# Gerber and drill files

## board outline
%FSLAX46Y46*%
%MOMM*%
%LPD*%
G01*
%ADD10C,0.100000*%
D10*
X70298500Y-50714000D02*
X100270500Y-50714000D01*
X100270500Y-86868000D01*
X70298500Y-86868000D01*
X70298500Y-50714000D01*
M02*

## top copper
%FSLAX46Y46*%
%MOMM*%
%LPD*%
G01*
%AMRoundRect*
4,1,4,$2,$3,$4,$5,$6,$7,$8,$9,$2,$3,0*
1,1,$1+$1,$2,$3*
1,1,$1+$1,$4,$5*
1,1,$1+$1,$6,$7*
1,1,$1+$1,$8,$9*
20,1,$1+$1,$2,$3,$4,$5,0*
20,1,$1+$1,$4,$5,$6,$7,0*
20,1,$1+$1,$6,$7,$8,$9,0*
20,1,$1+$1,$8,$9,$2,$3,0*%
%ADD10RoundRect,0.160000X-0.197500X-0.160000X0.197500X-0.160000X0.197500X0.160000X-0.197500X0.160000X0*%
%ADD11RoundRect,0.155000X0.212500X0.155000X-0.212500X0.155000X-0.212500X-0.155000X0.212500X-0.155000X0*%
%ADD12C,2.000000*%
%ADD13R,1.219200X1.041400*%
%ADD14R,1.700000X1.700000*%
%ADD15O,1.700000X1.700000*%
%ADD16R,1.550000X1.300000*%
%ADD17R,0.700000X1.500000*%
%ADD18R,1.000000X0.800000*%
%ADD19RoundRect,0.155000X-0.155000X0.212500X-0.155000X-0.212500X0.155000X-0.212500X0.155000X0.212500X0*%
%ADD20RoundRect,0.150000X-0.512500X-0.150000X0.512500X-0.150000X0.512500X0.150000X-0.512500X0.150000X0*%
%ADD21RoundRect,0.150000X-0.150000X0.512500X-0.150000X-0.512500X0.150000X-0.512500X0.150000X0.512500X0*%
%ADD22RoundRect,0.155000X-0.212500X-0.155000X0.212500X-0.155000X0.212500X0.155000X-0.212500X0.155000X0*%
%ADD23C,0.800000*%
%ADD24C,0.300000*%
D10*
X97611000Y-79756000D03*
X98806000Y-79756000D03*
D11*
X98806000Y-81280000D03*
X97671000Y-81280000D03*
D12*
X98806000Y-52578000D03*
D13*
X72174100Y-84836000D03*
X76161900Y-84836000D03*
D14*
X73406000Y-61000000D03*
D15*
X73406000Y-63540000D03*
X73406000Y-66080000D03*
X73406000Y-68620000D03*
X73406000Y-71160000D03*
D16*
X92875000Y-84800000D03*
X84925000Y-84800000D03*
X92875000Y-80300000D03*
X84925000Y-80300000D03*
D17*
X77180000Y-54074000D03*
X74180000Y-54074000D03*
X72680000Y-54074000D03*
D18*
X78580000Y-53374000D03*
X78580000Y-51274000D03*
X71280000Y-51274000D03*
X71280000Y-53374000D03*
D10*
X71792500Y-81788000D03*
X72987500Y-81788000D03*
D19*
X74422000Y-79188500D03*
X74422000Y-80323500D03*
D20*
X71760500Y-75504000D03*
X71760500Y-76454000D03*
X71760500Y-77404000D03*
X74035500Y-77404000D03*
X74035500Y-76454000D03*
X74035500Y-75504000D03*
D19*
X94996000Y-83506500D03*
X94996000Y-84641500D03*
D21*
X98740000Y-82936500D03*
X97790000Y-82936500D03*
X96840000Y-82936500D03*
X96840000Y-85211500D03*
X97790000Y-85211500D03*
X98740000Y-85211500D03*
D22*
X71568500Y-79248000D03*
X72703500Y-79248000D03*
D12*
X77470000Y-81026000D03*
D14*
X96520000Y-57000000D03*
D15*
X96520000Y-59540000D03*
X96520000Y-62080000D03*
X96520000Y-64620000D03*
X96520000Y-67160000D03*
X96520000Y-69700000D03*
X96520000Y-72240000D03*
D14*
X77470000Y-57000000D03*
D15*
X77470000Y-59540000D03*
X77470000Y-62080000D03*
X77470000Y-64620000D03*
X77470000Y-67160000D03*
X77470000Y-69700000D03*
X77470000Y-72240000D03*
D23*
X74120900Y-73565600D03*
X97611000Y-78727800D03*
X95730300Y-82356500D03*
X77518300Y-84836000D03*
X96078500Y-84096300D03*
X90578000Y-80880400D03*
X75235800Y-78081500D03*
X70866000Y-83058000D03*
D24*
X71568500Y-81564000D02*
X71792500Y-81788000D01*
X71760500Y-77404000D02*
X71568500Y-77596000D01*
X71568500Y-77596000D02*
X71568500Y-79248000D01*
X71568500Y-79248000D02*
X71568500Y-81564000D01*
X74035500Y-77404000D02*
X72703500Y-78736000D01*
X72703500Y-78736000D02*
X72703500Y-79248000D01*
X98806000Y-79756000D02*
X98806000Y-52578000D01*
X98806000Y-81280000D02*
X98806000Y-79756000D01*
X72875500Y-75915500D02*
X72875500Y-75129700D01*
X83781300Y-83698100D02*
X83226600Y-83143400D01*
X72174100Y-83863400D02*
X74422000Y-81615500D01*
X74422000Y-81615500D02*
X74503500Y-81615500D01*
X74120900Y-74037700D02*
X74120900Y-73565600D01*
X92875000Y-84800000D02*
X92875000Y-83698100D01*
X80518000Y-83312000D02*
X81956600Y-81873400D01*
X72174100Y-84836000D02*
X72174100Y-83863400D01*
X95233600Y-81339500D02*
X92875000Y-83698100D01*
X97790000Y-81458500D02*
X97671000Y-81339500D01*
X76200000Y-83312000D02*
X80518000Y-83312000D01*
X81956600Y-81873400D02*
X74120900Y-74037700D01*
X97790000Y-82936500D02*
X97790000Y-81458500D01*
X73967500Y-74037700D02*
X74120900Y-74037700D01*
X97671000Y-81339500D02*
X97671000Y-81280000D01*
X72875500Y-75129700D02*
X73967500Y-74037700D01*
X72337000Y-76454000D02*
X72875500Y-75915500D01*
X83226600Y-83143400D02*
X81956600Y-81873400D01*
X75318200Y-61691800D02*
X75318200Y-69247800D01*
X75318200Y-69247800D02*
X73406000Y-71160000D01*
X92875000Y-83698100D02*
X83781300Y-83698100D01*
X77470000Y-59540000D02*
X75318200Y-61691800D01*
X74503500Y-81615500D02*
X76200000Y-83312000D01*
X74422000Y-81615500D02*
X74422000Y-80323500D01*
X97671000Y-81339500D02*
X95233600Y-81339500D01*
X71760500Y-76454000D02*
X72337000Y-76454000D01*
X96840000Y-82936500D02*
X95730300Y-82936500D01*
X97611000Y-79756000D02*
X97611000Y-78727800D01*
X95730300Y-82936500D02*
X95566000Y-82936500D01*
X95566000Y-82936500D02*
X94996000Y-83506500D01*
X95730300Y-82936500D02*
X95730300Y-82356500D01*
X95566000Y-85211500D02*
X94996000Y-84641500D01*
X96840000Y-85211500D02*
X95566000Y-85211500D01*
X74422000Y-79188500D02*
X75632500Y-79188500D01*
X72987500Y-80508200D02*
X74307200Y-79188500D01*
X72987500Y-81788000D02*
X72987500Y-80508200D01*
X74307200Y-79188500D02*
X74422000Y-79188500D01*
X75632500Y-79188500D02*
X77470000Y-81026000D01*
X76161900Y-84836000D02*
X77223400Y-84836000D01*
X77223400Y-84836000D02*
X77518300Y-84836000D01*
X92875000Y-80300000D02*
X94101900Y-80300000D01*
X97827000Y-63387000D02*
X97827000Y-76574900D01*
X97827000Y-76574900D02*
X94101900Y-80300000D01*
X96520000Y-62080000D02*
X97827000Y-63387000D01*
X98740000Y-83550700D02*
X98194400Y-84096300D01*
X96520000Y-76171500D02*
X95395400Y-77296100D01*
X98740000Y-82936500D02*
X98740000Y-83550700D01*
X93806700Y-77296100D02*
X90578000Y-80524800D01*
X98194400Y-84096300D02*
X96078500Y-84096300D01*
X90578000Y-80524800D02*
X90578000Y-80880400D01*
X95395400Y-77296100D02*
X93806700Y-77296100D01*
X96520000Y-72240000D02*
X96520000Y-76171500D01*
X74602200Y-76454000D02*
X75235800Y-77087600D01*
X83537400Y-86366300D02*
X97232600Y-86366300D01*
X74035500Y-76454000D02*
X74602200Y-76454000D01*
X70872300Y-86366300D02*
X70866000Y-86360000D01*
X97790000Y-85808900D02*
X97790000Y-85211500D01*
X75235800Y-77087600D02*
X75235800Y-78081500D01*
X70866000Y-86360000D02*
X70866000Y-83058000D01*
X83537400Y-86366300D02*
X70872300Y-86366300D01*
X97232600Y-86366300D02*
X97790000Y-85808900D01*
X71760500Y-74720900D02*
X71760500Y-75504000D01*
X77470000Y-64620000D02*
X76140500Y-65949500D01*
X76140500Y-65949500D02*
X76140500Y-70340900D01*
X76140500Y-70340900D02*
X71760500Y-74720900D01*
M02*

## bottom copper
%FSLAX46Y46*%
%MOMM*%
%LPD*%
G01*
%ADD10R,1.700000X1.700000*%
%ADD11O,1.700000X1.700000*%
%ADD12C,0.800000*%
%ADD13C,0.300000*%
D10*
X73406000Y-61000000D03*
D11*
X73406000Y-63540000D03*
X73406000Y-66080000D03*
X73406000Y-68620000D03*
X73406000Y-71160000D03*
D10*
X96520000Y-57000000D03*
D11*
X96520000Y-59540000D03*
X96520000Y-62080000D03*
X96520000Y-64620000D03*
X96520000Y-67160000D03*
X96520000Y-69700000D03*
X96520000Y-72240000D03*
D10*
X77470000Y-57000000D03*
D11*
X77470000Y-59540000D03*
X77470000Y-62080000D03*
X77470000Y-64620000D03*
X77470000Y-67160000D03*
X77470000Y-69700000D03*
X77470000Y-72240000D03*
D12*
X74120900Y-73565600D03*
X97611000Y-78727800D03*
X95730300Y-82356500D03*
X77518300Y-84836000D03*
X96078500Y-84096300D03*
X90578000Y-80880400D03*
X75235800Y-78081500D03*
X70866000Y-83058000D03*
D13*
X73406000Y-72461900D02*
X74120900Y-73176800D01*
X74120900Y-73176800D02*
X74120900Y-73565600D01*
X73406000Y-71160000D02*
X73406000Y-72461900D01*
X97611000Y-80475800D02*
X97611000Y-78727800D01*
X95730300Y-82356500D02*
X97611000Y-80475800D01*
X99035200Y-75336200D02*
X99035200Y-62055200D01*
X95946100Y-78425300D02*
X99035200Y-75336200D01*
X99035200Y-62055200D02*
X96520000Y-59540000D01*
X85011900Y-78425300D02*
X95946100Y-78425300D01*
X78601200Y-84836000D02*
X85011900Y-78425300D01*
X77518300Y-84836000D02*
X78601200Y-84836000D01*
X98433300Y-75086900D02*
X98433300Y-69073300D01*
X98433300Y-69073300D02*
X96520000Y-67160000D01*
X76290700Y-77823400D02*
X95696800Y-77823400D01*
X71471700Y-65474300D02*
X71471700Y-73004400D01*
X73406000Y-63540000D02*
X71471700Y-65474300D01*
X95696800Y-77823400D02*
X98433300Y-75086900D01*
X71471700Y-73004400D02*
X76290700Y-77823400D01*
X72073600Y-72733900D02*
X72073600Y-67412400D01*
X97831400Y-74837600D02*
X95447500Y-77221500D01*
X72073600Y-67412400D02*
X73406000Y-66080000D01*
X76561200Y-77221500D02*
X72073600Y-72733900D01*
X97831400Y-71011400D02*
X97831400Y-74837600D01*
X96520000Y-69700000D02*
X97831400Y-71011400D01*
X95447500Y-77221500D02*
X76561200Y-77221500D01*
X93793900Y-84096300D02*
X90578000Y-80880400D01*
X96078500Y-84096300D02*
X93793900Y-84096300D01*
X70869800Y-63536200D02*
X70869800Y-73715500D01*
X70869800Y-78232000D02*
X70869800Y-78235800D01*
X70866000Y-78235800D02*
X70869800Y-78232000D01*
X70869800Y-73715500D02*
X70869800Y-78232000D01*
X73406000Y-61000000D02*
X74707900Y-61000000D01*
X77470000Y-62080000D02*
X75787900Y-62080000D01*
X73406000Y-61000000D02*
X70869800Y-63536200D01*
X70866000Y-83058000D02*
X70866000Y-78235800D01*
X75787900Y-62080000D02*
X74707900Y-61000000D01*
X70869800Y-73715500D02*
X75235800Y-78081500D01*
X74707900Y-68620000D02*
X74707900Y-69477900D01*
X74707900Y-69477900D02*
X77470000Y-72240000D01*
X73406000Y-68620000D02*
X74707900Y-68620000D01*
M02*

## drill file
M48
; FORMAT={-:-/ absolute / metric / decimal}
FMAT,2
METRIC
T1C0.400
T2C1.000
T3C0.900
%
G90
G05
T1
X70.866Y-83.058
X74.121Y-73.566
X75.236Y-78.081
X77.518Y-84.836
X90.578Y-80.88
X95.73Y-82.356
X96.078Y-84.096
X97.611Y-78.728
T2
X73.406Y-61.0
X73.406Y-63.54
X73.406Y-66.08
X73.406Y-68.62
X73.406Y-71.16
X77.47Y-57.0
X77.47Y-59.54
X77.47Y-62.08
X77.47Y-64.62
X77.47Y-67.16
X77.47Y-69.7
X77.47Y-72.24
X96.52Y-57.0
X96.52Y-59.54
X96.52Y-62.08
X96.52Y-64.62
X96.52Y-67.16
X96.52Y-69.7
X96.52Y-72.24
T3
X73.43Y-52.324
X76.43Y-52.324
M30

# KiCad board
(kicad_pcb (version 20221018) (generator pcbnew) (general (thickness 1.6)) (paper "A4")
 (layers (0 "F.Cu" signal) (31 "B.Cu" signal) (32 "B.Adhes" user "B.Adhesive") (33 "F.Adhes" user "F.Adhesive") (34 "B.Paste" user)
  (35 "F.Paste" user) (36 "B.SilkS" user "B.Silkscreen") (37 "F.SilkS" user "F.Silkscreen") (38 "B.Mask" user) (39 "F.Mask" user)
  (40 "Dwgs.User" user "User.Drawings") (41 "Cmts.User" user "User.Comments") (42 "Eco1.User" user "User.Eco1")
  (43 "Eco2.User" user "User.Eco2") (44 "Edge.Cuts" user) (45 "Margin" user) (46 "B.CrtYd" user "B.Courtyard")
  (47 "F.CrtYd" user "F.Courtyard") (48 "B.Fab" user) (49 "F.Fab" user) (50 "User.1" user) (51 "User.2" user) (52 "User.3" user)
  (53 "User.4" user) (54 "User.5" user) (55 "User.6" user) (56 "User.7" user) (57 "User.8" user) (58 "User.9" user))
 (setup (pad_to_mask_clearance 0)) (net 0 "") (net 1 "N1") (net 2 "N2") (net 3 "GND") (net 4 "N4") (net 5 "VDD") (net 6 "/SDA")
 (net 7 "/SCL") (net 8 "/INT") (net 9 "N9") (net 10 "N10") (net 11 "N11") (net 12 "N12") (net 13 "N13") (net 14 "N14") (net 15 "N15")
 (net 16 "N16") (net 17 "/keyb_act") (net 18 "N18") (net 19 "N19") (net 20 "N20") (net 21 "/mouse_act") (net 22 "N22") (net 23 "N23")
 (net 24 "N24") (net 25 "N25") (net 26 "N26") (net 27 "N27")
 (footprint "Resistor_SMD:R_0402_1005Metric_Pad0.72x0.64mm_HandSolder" (layer "F.Cu") (at 98.2085 79.756)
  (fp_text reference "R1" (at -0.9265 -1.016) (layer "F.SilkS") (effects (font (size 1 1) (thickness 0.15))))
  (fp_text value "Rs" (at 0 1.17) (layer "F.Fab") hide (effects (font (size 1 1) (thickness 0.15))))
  (pad "1" smd roundrect (at -0.5975 0) (size 0.715 0.64) (layers "F.Cu" "F.Paste" "F.Mask") (roundrect_rratio 0.25) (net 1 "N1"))
  (pad "2" smd roundrect (at 0.5975 0) (size 0.715 0.64) (layers "F.Cu" "F.Paste" "F.Mask") (roundrect_rratio 0.25) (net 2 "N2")))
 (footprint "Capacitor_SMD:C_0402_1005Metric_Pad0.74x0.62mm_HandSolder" (layer "F.Cu") (at 98.2385 81.28 180)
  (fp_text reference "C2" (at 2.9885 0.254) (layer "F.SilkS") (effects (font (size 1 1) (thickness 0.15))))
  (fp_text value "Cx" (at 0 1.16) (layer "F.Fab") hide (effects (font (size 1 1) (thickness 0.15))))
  (pad "1" smd roundrect (at -0.5675 0 180) (size 0.735 0.62) (layers "F.Cu" "F.Paste" "F.Mask") (roundrect_rratio 0.25) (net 2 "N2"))
  (pad "2" smd roundrect (at 0.5675 0 180) (size 0.735 0.62) (layers "F.Cu" "F.Paste" "F.Mask") (roundrect_rratio 0.25) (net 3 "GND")))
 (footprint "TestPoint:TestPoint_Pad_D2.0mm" (layer "F.Cu") (at 98.806 52.578)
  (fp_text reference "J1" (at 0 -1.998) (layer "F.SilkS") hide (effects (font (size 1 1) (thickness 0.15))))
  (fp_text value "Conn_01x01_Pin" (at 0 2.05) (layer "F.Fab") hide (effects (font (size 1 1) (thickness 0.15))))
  (pad "1" smd circle (at 0 0) (size 2 2) (layers "F.Cu" "F.Mask") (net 2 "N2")))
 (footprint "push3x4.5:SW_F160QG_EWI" (layer "F.Cu") (at 74.168 84.836)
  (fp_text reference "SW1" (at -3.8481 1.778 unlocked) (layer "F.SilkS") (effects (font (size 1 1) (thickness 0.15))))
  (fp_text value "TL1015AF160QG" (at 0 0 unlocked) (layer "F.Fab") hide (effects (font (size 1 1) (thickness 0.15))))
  (pad "1" smd rect (at -1.9939 0) (size 1.2192 1.0414) (layers "F.Cu" "F.Paste" "F.Mask") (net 3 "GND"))
  (pad "2" smd rect (at 1.9939 0) (size 1.2192 1.0414) (layers "F.Cu" "F.Paste" "F.Mask") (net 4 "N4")))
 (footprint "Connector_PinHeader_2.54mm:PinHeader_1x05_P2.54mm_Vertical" (layer "F.Cu") (at 73.406 61)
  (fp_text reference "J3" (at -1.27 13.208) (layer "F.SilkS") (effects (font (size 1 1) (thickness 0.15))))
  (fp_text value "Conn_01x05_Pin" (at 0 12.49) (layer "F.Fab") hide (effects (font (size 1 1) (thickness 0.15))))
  (pad "1" thru_hole rect (at 0 0) (size 1.7 1.7) (drill 1) (layers "*.Cu" "*.Mask") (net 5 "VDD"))
  (pad "2" thru_hole oval (at 0 2.54) (size 1.7 1.7) (drill 1) (layers "*.Cu" "*.Mask") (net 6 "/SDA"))
  (pad "3" thru_hole oval (at 0 5.08) (size 1.7 1.7) (drill 1) (layers "*.Cu" "*.Mask") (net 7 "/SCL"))
  (pad "4" thru_hole oval (at 0 7.62) (size 1.7 1.7) (drill 1) (layers "*.Cu" "*.Mask") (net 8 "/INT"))
  (pad "5" thru_hole oval (at 0 10.16) (size 1.7 1.7) (drill 1) (layers "*.Cu" "*.Mask") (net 3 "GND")))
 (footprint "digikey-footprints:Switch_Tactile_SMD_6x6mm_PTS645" (layer "F.Cu") (at 88.9 82.55 180)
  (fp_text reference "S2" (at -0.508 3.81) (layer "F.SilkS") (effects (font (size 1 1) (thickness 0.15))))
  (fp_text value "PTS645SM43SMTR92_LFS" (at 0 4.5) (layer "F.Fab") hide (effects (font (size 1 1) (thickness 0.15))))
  (pad "1" smd rect (at -3.975 -2.25 180) (size 1.55 1.3) (layers "F.Cu" "F.Paste" "F.Mask") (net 3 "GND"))
  (pad "2" smd rect (at 3.975 -2.25 180) (size 1.55 1.3) (layers "F.Cu" "F.Paste" "F.Mask") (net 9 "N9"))
  (pad "3" smd rect (at -3.975 2.25 180) (size 1.55 1.3) (layers "F.Cu" "F.Paste" "F.Mask") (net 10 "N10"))
  (pad "4" smd rect (at 3.975 2.25 180) (size 1.55 1.3) (layers "F.Cu" "F.Paste" "F.Mask") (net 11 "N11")))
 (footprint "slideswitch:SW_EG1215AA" (layer "F.Cu") (at 74.93 52.324 180)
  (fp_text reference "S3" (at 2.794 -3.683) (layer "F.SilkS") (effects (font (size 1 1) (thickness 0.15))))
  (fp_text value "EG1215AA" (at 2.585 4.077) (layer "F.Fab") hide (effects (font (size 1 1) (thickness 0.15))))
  (pad "" np_thru_hole circle (at -1.5 0 180) (size 0.9 0.9) (drill 0.9) (layers "*.Cu" "*.Mask"))
  (pad "" np_thru_hole circle (at 1.5 0 180) (size 0.9 0.9) (drill 0.9) (layers "*.Cu" "*.Mask"))
  (pad "1" smd rect (at -2.25 -1.75 180) (size 0.7 1.5) (layers "F.Cu" "F.Paste" "F.Mask") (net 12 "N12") (solder_mask_margin 0.102))
  (pad "2" smd rect (at 0.75 -1.75 180) (size 0.7 1.5) (layers "F.Cu" "F.Paste" "F.Mask") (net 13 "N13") (solder_mask_margin 0.102))
  (pad "3" smd rect (at 2.25 -1.75 180) (size 0.7 1.5) (layers "F.Cu" "F.Paste" "F.Mask") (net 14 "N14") (solder_mask_margin 0.102))
  (pad "S1" smd rect (at -3.65 -1.05 180) (size 1 0.8) (layers "F.Cu" "F.Paste" "F.Mask") (solder_mask_margin 0.102))
  (pad "S2" smd rect (at -3.65 1.05 180) (size 1 0.8) (layers "F.Cu" "F.Paste" "F.Mask") (solder_mask_margin 0.102))
  (pad "S3" smd rect (at 3.65 1.05 180) (size 1 0.8) (layers "F.Cu" "F.Paste" "F.Mask") (solder_mask_margin 0.102))
  (pad "S4" smd rect (at 3.65 -1.05 180) (size 1 0.8) (layers "F.Cu" "F.Paste" "F.Mask") (solder_mask_margin 0.102)))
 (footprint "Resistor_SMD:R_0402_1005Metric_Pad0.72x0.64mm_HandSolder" (layer "F.Cu") (at 72.39 81.788)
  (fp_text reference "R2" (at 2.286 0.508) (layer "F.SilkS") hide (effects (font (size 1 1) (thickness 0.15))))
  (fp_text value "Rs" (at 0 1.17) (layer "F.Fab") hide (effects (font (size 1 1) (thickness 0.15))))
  (pad "1" smd roundrect (at -0.5975 0) (size 0.715 0.64) (layers "F.Cu" "F.Paste" "F.Mask") (roundrect_rratio 0.25) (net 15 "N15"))
  (pad "2" smd roundrect (at 0.5975 0) (size 0.715 0.64) (layers "F.Cu" "F.Paste" "F.Mask") (roundrect_rratio 0.25) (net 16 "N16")))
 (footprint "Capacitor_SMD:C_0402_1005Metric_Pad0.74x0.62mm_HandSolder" (layer "F.Cu") (at 74.422 79.756 -90)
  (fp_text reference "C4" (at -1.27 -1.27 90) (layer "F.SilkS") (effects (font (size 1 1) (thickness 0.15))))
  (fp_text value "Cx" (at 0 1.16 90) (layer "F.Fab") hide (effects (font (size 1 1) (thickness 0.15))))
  (pad "1" smd roundrect (at -0.5675 0 270) (size 0.735 0.62) (layers "F.Cu" "F.Paste" "F.Mask") (roundrect_rratio 0.25) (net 16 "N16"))
  (pad "2" smd roundrect (at 0.5675 0 270) (size 0.735 0.62) (layers "F.Cu" "F.Paste" "F.Mask") (roundrect_rratio 0.25) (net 3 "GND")))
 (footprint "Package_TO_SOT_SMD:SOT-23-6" (layer "F.Cu") (at 72.898 76.454)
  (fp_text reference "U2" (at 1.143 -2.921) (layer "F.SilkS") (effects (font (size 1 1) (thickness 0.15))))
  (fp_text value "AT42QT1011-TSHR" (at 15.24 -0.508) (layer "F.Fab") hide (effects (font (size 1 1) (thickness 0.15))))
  (pad "1" smd roundrect (at -1.1375 -0.95) (size 1.325 0.6) (layers "F.Cu" "F.Paste" "F.Mask") (roundrect_rratio 0.25) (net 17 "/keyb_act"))
  (pad "2" smd roundrect (at -1.1375 0) (size 1.325 0.6) (layers "F.Cu" "F.Paste" "F.Mask") (roundrect_rratio 0.25) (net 3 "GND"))
  (pad "3" smd roundrect (at -1.1375 0.95) (size 1.325 0.6) (layers "F.Cu" "F.Paste" "F.Mask") (roundrect_rratio 0.25) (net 15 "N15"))
  (pad "4" smd roundrect (at 1.1375 0.95) (size 1.325 0.6) (layers "F.Cu" "F.Paste" "F.Mask") (roundrect_rratio 0.25) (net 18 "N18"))
  (pad "5" smd roundrect (at 1.1375 0) (size 1.325 0.6) (layers "F.Cu" "F.Paste" "F.Mask") (roundrect_rratio 0.25) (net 5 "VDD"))
  (pad "6" smd roundrect (at 1.1375 -0.95) (size 1.325 0.6) (layers "F.Cu" "F.Paste" "F.Mask") (roundrect_rratio 0.25) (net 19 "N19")))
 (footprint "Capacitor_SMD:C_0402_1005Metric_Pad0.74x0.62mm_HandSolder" (layer "F.Cu") (at 94.996 84.074 -90)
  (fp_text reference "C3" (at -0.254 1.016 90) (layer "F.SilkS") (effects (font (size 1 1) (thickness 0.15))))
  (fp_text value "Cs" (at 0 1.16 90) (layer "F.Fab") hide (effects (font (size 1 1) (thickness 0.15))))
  (pad "1" smd roundrect (at -0.5675 0 270) (size 0.735 0.62) (layers "F.Cu" "F.Paste" "F.Mask") (roundrect_rratio 0.25) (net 1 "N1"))
  (pad "2" smd roundrect (at 0.5675 0 270) (size 0.735 0.62) (layers "F.Cu" "F.Paste" "F.Mask") (roundrect_rratio 0.25) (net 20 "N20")))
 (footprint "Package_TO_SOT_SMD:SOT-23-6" (layer "F.Cu") (at 97.79 84.074 -90)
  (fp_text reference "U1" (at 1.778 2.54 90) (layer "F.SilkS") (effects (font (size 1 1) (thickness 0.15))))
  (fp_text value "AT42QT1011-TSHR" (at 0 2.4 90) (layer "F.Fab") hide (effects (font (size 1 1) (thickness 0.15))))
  (pad "1" smd roundrect (at -1.1375 -0.95 270) (size 1.325 0.6) (layers "F.Cu" "F.Paste" "F.Mask") (roundrect_rratio 0.25)
   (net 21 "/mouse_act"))
  (pad "2" smd roundrect (at -1.1375 0 270) (size 1.325 0.6) (layers "F.Cu" "F.Paste" "F.Mask") (roundrect_rratio 0.25) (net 3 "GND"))
  (pad "3" smd roundrect (at -1.1375 0.95 270) (size 1.325 0.6) (layers "F.Cu" "F.Paste" "F.Mask") (roundrect_rratio 0.25) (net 1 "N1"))
  (pad "4" smd roundrect (at 1.1375 0.95 270) (size 1.325 0.6) (layers "F.Cu" "F.Paste" "F.Mask") (roundrect_rratio 0.25) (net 20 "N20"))
  (pad "5" smd roundrect (at 1.1375 0 270) (size 1.325 0.6) (layers "F.Cu" "F.Paste" "F.Mask") (roundrect_rratio 0.25) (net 5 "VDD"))
  (pad "6" smd roundrect (at 1.1375 -0.95 270) (size 1.325 0.6) (layers "F.Cu" "F.Paste" "F.Mask") (roundrect_rratio 0.25) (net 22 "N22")))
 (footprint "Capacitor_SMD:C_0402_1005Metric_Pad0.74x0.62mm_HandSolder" (layer "F.Cu") (at 72.136 79.248)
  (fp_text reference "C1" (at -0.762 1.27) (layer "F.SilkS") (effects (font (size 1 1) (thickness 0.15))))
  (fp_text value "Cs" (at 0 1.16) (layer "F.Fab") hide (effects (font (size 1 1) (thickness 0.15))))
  (pad "1" smd roundrect (at -0.5675 0) (size 0.735 0.62) (layers "F.Cu" "F.Paste" "F.Mask") (roundrect_rratio 0.25) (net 15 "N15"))
  (pad "2" smd roundrect (at 0.5675 0) (size 0.735 0.62) (layers "F.Cu" "F.Paste" "F.Mask") (roundrect_rratio 0.25) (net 18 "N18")))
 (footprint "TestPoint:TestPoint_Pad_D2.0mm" (layer "F.Cu") (at 77.47 81.026)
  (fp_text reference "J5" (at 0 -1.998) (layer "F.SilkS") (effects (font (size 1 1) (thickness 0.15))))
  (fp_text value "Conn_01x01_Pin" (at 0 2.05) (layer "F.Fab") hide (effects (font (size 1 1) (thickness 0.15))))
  (pad "1" smd circle (at 0 0) (size 2 2) (layers "F.Cu" "F.Mask") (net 16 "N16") (clearance 1)))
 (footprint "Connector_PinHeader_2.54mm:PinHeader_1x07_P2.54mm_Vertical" (layer "B.Cu") (at 96.52 57 180)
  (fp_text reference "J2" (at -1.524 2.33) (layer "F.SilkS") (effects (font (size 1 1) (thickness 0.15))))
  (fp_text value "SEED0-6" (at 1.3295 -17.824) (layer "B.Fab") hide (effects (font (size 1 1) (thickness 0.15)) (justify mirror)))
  (pad "1" thru_hole rect (at 0 0 180) (size 1.7 1.7) (drill 1) (layers "*.Cu" "*.Mask") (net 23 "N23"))
  (pad "2" thru_hole oval (at 0 -2.54 180) (size 1.7 1.7) (drill 1) (layers "*.Cu" "*.Mask") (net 4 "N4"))
  (pad "3" thru_hole oval (at 0 -5.08 180) (size 1.7 1.7) (drill 1) (layers "*.Cu" "*.Mask") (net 10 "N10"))
  (pad "4" thru_hole oval (at 0 -7.62 180) (size 1.7 1.7) (drill 1) (layers "*.Cu" "*.Mask") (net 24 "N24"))
  (pad "5" thru_hole oval (at 0 -10.16 180) (size 1.7 1.7) (drill 1) (layers "*.Cu" "*.Mask") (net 6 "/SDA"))
  (pad "6" thru_hole oval (at 0 -12.7 180) (size 1.7 1.7) (drill 1) (layers "*.Cu" "*.Mask") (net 7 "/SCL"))
  (pad "7" thru_hole oval (at 0 -15.24 180) (size 1.7 1.7) (drill 1) (layers "*.Cu" "*.Mask") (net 21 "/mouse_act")))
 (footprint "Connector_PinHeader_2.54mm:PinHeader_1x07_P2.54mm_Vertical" (layer "B.Cu") (at 77.47 57 180)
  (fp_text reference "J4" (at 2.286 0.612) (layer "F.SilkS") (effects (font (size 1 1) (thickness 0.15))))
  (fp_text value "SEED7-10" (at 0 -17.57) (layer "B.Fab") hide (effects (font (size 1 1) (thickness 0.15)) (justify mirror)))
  (pad "1" thru_hole rect (at 0 0 180) (size 1.7 1.7) (drill 1) (layers "*.Cu" "*.Mask") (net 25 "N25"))
  (pad "2" thru_hole oval (at 0 -2.54 180) (size 1.7 1.7) (drill 1) (layers "*.Cu" "*.Mask") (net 3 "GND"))
  (pad "3" thru_hole oval (at 0 -5.08 180) (size 1.7 1.7) (drill 1) (layers "*.Cu" "*.Mask") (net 5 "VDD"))
  (pad "4" thru_hole oval (at 0 -7.62 180) (size 1.7 1.7) (drill 1) (layers "*.Cu" "*.Mask") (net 17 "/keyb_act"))
  (pad "5" thru_hole oval (at 0 -10.16 180) (size 1.7 1.7) (drill 1) (layers "*.Cu" "*.Mask") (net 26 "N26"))
  (pad "6" thru_hole oval (at 0 -12.7 180) (size 1.7 1.7) (drill 1) (layers "*.Cu" "*.Mask") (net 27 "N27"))
  (pad "7" thru_hole oval (at 0 -15.24 180) (size 1.7 1.7) (drill 1) (layers "*.Cu" "*.Mask") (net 8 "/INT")))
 (gr_rect (start 70.2985 50.714) (end 100.2705 86.868) (stroke (width 0.1) (type default)) (fill none) (layer "Edge.Cuts"))
 (segment (start 71.5685 81.564) (end 71.7925 81.788) (width 0.3) (layer "F.Cu") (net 15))
 (segment (start 71.7605 77.404) (end 71.5685 77.596) (width 0.3) (layer "F.Cu") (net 15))
 (segment (start 71.5685 77.596) (end 71.5685 79.248) (width 0.3) (layer "F.Cu") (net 15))
 (segment (start 71.5685 79.248) (end 71.5685 81.564) (width 0.3) (layer "F.Cu") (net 15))
 (segment (start 74.0355 77.404) (end 72.7035 78.736) (width 0.3) (layer "F.Cu") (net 18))
 (segment (start 72.7035 78.736) (end 72.7035 79.248) (width 0.3) (layer "F.Cu") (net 18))
 (segment (start 98.806 79.756) (end 98.806 52.578) (width 0.3) (layer "F.Cu") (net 2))
 (segment (start 98.806 81.28) (end 98.806 79.756) (width 0.3) (layer "F.Cu") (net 2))
 (segment (start 72.8755 75.9155) (end 72.8755 75.1297) (width 0.3) (layer "F.Cu") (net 3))
 (segment (start 83.7813 83.6981) (end 83.2266 83.1434) (width 0.3) (layer "F.Cu") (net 3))
 (segment (start 72.1741 83.8634) (end 74.422 81.6155) (width 0.3) (layer "F.Cu") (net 3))
 (segment (start 74.422 81.6155) (end 74.5035 81.6155) (width 0.3) (layer "F.Cu") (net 3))
 (segment (start 74.1209 74.0377) (end 74.1209 73.5656) (width 0.3) (layer "F.Cu") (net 3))
 (segment (start 92.875 84.8) (end 92.875 83.6981) (width 0.3) (layer "F.Cu") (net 3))
 (segment (start 80.518 83.312) (end 81.9566 81.8734) (width 0.3) (layer "F.Cu") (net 3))
 (segment (start 72.1741 84.836) (end 72.1741 83.8634) (width 0.3) (layer "F.Cu") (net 3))
 (segment (start 95.2336 81.3395) (end 92.875 83.6981) (width 0.3) (layer "F.Cu") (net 3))
 (segment (start 97.79 81.4585) (end 97.671 81.3395) (width 0.3) (layer "F.Cu") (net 3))
 (segment (start 76.2 83.312) (end 80.518 83.312) (width 0.3) (layer "F.Cu") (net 3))
 (segment (start 81.9566 81.8734) (end 74.1209 74.0377) (width 0.3) (layer "F.Cu") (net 3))
 (segment (start 97.79 82.9365) (end 97.79 81.4585) (width 0.3) (layer "F.Cu") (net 3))
 (segment (start 73.9675 74.0377) (end 74.1209 74.0377) (width 0.3) (layer "F.Cu") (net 3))
 (segment (start 97.671 81.3395) (end 97.671 81.28) (width 0.3) (layer "F.Cu") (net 3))
 (segment (start 72.8755 75.1297) (end 73.9675 74.0377) (width 0.3) (layer "F.Cu") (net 3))
 (segment (start 72.337 76.454) (end 72.8755 75.9155) (width 0.3) (layer "F.Cu") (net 3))
 (segment (start 83.2266 83.1434) (end 81.9566 81.8734) (width 0.3) (layer "F.Cu") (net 3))
 (segment (start 75.3182 61.6918) (end 75.3182 69.2478) (width 0.3) (layer "F.Cu") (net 3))
 (segment (start 75.3182 69.2478) (end 73.406 71.16) (width 0.3) (layer "F.Cu") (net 3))
 (segment (start 92.875 83.6981) (end 83.7813 83.6981) (width 0.3) (layer "F.Cu") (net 3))
 (segment (start 77.47 59.54) (end 75.3182 61.6918) (width 0.3) (layer "F.Cu") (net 3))
 (segment (start 74.5035 81.6155) (end 76.2 83.312) (width 0.3) (layer "F.Cu") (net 3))
 (segment (start 74.422 81.6155) (end 74.422 80.3235) (width 0.3) (layer "F.Cu") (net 3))
 (segment (start 97.671 81.3395) (end 95.2336 81.3395) (width 0.3) (layer "F.Cu") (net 3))
 (segment (start 71.7605 76.454) (end 72.337 76.454) (width 0.3) (layer "F.Cu") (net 3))
 (via (at 74.1209 73.5656) (size 0.8) (drill 0.4) (layers "F.Cu" "B.Cu") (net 3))
 (segment (start 73.406 72.4619) (end 74.1209 73.1768) (width 0.3) (layer "B.Cu") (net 3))
 (segment (start 74.1209 73.1768) (end 74.1209 73.5656) (width 0.3) (layer "B.Cu") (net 3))
 (segment (start 73.406 71.16) (end 73.406 72.4619) (width 0.3) (layer "B.Cu") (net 3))
 (segment (start 96.84 82.9365) (end 95.7303 82.9365) (width 0.3) (layer "F.Cu") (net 1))
 (segment (start 97.611 79.756) (end 97.611 78.7278) (width 0.3) (layer "F.Cu") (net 1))
 (segment (start 95.7303 82.9365) (end 95.566 82.9365) (width 0.3) (layer "F.Cu") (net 1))
 (segment (start 95.566 82.9365) (end 94.996 83.5065) (width 0.3) (layer "F.Cu") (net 1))
 (segment (start 95.7303 82.9365) (end 95.7303 82.3565) (width 0.3) (layer "F.Cu") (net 1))
 (via (at 97.611 78.7278) (size 0.8) (drill 0.4) (layers "F.Cu" "B.Cu") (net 1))
 (via (at 95.7303 82.3565) (size 0.8) (drill 0.4) (layers "F.Cu" "B.Cu") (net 1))
 (segment (start 97.611 80.4758) (end 97.611 78.7278) (width 0.3) (layer "B.Cu") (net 1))
 (segment (start 95.7303 82.3565) (end 97.611 80.4758) (width 0.3) (layer "B.Cu") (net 1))
 (segment (start 95.566 85.2115) (end 94.996 84.6415) (width 0.3) (layer "F.Cu") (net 20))
 (segment (start 96.84 85.2115) (end 95.566 85.2115) (width 0.3) (layer "F.Cu") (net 20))
 (segment (start 74.422 79.1885) (end 75.6325 79.1885) (width 0.3) (layer "F.Cu") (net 16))
 (segment (start 72.9875 80.5082) (end 74.3072 79.1885) (width 0.3) (layer "F.Cu") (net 16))
 (segment (start 72.9875 81.788) (end 72.9875 80.5082) (width 0.3) (layer "F.Cu") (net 16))
 (segment (start 74.3072 79.1885) (end 74.422 79.1885) (width 0.3) (layer "F.Cu") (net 16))
 (segment (start 75.6325 79.1885) (end 77.47 81.026) (width 0.3) (layer "F.Cu") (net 16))
 (segment (start 76.1619 84.836) (end 77.2234 84.836) (width 0.3) (layer "F.Cu") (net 4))
 (segment (start 77.2234 84.836) (end 77.5183 84.836) (width 0.3) (layer "F.Cu") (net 4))
 (via (at 77.5183 84.836) (size 0.8) (drill 0.4) (layers "F.Cu" "B.Cu") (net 4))
 (segment (start 99.0352 75.3362) (end 99.0352 62.0552) (width 0.3) (layer "B.Cu") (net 4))
 (segment (start 95.9461 78.4253) (end 99.0352 75.3362) (width 0.3) (layer "B.Cu") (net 4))
 (segment (start 99.0352 62.0552) (end 96.52 59.54) (width 0.3) (layer "B.Cu") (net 4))
 (segment (start 85.0119 78.4253) (end 95.9461 78.4253) (width 0.3) (layer "B.Cu") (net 4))
 (segment (start 78.6012 84.836) (end 85.0119 78.4253) (width 0.3) (layer "B.Cu") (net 4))
 (segment (start 77.5183 84.836) (end 78.6012 84.836) (width 0.3) (layer "B.Cu") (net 4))
 (segment (start 92.875 80.3) (end 94.1019 80.3) (width 0.3) (layer "F.Cu") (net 10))
 (segment (start 97.827 63.387) (end 97.827 76.5749) (width 0.3) (layer "F.Cu") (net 10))
 (segment (start 97.827 76.5749) (end 94.1019 80.3) (width 0.3) (layer "F.Cu") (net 10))
 (segment (start 96.52 62.08) (end 97.827 63.387) (width 0.3) (layer "F.Cu") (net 10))
 (segment (start 98.4333 75.0869) (end 98.4333 69.0733) (width 0.3) (layer "B.Cu") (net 6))
 (segment (start 98.4333 69.0733) (end 96.52 67.16) (width 0.3) (layer "B.Cu") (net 6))
 (segment (start 76.2907 77.8234) (end 95.6968 77.8234) (width 0.3) (layer "B.Cu") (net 6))
 (segment (start 71.4717 65.4743) (end 71.4717 73.0044) (width 0.3) (layer "B.Cu") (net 6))
 (segment (start 73.406 63.54) (end 71.4717 65.4743) (width 0.3) (layer "B.Cu") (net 6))
 (segment (start 95.6968 77.8234) (end 98.4333 75.0869) (width 0.3) (layer "B.Cu") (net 6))
 (segment (start 71.4717 73.0044) (end 76.2907 77.8234) (width 0.3) (layer "B.Cu") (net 6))
 (segment (start 72.0736 72.7339) (end 72.0736 67.4124) (width 0.3) (layer "B.Cu") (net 7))
 (segment (start 97.8314 74.8376) (end 95.4475 77.2215) (width 0.3) (layer "B.Cu") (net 7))
 (segment (start 72.0736 67.4124) (end 73.406 66.08) (width 0.3) (layer "B.Cu") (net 7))
 (segment (start 76.5612 77.2215) (end 72.0736 72.7339) (width 0.3) (layer "B.Cu") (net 7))
 (segment (start 97.8314 71.0114) (end 97.8314 74.8376) (width 0.3) (layer "B.Cu") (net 7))
 (segment (start 96.52 69.7) (end 97.8314 71.0114) (width 0.3) (layer "B.Cu") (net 7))
 (segment (start 95.4475 77.2215) (end 76.5612 77.2215) (width 0.3) (layer "B.Cu") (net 7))
 (segment (start 98.74 83.5507) (end 98.1944 84.0963) (width 0.3) (layer "F.Cu") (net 21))
 (segment (start 96.52 76.1715) (end 95.3954 77.2961) (width 0.3) (layer "F.Cu") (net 21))
 (segment (start 98.74 82.9365) (end 98.74 83.5507) (width 0.3) (layer "F.Cu") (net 21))
 (segment (start 93.8067 77.2961) (end 90.578 80.5248) (width 0.3) (layer "F.Cu") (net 21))
 (segment (start 98.1944 84.0963) (end 96.0785 84.0963) (width 0.3) (layer "F.Cu") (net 21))
 (segment (start 90.578 80.5248) (end 90.578 80.8804) (width 0.3) (layer "F.Cu") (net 21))
 (segment (start 95.3954 77.2961) (end 93.8067 77.2961) (width 0.3) (layer "F.Cu") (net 21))
 (segment (start 96.52 72.24) (end 96.52 76.1715) (width 0.3) (layer "F.Cu") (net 21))
 (via (at 96.0785 84.0963) (size 0.8) (drill 0.4) (layers "F.Cu" "B.Cu") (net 21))
 (via (at 90.578 80.8804) (size 0.8) (drill 0.4) (layers "F.Cu" "B.Cu") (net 21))
 (segment (start 93.7939 84.0963) (end 90.578 80.8804) (width 0.3) (layer "B.Cu") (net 21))
 (segment (start 96.0785 84.0963) (end 93.7939 84.0963) (width 0.3) (layer "B.Cu") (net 21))
 (segment (start 74.6022 76.454) (end 75.2358 77.0876) (width 0.3) (layer "F.Cu") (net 5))
 (segment (start 83.5374 86.3663) (end 97.2326 86.3663) (width 0.3) (layer "F.Cu") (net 5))
 (segment (start 74.0355 76.454) (end 74.6022 76.454) (width 0.3) (layer "F.Cu") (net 5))
 (segment (start 70.8723 86.3663) (end 70.866 86.36) (width 0.3) (layer "F.Cu") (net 5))
 (segment (start 97.79 85.8089) (end 97.79 85.2115) (width 0.3) (layer "F.Cu") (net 5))
 (segment (start 75.2358 77.0876) (end 75.2358 78.0815) (width 0.3) (layer "F.Cu") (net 5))
 (segment (start 70.866 86.36) (end 70.866 83.058) (width 0.3) (layer "F.Cu") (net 5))
 (segment (start 83.5374 86.3663) (end 70.8723 86.3663) (width 0.3) (layer "F.Cu") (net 5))
 (segment (start 97.2326 86.3663) (end 97.79 85.8089) (width 0.3) (layer "F.Cu") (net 5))
 (via (at 75.2358 78.0815) (size 0.8) (drill 0.4) (layers "F.Cu" "B.Cu") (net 5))
 (via (at 70.866 83.058) (size 0.8) (drill 0.4) (layers "F.Cu" "B.Cu") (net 5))
 (segment (start 70.8698 63.5362) (end 70.8698 73.7155) (width 0.3) (layer "B.Cu") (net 5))
 (segment (start 70.8698 78.232) (end 70.8698 78.2358) (width 0.3) (layer "B.Cu") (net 5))
 (segment (start 70.866 78.2358) (end 70.8698 78.232) (width 0.3) (layer "B.Cu") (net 5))
 (segment (start 70.8698 73.7155) (end 70.8698 78.232) (width 0.3) (layer "B.Cu") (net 5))
 (segment (start 73.406 61) (end 74.7079 61) (width 0.3) (layer "B.Cu") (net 5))
 (segment (start 77.47 62.08) (end 75.7879 62.08) (width 0.3) (layer "B.Cu") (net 5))
 (segment (start 73.406 61) (end 70.8698 63.5362) (width 0.3) (layer "B.Cu") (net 5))
 (segment (start 70.866 83.058) (end 70.866 78.2358) (width 0.3) (layer "B.Cu") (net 5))
 (segment (start 75.7879 62.08) (end 74.7079 61) (width 0.3) (layer "B.Cu") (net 5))
 (segment (start 70.8698 73.7155) (end 75.2358 78.0815) (width 0.3) (layer "B.Cu") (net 5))
 (segment (start 74.7079 68.62) (end 74.7079 69.4779) (width 0.3) (layer "B.Cu") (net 8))
 (segment (start 74.7079 69.4779) (end 77.47 72.24) (width 0.3) (layer "B.Cu") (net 8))
 (segment (start 73.406 68.62) (end 74.7079 68.62) (width 0.3) (layer "B.Cu") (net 8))
 (segment (start 71.7605 74.7209) (end 71.7605 75.504) (width 0.3) (layer "F.Cu") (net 17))
 (segment (start 77.47 64.62) (end 76.1405 65.9495) (width 0.3) (layer "F.Cu") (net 17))
 (segment (start 76.1405 65.9495) (end 76.1405 70.3409) (width 0.3) (layer "F.Cu") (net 17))
 (segment (start 76.1405 70.3409) (end 71.7605 74.7209) (width 0.3) (layer "F.Cu") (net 17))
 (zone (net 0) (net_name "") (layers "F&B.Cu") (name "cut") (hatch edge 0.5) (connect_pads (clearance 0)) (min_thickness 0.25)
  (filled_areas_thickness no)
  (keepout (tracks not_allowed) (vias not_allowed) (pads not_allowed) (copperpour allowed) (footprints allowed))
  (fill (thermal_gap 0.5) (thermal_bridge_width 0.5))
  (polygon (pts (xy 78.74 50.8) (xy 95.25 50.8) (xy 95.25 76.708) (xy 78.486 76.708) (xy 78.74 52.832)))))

